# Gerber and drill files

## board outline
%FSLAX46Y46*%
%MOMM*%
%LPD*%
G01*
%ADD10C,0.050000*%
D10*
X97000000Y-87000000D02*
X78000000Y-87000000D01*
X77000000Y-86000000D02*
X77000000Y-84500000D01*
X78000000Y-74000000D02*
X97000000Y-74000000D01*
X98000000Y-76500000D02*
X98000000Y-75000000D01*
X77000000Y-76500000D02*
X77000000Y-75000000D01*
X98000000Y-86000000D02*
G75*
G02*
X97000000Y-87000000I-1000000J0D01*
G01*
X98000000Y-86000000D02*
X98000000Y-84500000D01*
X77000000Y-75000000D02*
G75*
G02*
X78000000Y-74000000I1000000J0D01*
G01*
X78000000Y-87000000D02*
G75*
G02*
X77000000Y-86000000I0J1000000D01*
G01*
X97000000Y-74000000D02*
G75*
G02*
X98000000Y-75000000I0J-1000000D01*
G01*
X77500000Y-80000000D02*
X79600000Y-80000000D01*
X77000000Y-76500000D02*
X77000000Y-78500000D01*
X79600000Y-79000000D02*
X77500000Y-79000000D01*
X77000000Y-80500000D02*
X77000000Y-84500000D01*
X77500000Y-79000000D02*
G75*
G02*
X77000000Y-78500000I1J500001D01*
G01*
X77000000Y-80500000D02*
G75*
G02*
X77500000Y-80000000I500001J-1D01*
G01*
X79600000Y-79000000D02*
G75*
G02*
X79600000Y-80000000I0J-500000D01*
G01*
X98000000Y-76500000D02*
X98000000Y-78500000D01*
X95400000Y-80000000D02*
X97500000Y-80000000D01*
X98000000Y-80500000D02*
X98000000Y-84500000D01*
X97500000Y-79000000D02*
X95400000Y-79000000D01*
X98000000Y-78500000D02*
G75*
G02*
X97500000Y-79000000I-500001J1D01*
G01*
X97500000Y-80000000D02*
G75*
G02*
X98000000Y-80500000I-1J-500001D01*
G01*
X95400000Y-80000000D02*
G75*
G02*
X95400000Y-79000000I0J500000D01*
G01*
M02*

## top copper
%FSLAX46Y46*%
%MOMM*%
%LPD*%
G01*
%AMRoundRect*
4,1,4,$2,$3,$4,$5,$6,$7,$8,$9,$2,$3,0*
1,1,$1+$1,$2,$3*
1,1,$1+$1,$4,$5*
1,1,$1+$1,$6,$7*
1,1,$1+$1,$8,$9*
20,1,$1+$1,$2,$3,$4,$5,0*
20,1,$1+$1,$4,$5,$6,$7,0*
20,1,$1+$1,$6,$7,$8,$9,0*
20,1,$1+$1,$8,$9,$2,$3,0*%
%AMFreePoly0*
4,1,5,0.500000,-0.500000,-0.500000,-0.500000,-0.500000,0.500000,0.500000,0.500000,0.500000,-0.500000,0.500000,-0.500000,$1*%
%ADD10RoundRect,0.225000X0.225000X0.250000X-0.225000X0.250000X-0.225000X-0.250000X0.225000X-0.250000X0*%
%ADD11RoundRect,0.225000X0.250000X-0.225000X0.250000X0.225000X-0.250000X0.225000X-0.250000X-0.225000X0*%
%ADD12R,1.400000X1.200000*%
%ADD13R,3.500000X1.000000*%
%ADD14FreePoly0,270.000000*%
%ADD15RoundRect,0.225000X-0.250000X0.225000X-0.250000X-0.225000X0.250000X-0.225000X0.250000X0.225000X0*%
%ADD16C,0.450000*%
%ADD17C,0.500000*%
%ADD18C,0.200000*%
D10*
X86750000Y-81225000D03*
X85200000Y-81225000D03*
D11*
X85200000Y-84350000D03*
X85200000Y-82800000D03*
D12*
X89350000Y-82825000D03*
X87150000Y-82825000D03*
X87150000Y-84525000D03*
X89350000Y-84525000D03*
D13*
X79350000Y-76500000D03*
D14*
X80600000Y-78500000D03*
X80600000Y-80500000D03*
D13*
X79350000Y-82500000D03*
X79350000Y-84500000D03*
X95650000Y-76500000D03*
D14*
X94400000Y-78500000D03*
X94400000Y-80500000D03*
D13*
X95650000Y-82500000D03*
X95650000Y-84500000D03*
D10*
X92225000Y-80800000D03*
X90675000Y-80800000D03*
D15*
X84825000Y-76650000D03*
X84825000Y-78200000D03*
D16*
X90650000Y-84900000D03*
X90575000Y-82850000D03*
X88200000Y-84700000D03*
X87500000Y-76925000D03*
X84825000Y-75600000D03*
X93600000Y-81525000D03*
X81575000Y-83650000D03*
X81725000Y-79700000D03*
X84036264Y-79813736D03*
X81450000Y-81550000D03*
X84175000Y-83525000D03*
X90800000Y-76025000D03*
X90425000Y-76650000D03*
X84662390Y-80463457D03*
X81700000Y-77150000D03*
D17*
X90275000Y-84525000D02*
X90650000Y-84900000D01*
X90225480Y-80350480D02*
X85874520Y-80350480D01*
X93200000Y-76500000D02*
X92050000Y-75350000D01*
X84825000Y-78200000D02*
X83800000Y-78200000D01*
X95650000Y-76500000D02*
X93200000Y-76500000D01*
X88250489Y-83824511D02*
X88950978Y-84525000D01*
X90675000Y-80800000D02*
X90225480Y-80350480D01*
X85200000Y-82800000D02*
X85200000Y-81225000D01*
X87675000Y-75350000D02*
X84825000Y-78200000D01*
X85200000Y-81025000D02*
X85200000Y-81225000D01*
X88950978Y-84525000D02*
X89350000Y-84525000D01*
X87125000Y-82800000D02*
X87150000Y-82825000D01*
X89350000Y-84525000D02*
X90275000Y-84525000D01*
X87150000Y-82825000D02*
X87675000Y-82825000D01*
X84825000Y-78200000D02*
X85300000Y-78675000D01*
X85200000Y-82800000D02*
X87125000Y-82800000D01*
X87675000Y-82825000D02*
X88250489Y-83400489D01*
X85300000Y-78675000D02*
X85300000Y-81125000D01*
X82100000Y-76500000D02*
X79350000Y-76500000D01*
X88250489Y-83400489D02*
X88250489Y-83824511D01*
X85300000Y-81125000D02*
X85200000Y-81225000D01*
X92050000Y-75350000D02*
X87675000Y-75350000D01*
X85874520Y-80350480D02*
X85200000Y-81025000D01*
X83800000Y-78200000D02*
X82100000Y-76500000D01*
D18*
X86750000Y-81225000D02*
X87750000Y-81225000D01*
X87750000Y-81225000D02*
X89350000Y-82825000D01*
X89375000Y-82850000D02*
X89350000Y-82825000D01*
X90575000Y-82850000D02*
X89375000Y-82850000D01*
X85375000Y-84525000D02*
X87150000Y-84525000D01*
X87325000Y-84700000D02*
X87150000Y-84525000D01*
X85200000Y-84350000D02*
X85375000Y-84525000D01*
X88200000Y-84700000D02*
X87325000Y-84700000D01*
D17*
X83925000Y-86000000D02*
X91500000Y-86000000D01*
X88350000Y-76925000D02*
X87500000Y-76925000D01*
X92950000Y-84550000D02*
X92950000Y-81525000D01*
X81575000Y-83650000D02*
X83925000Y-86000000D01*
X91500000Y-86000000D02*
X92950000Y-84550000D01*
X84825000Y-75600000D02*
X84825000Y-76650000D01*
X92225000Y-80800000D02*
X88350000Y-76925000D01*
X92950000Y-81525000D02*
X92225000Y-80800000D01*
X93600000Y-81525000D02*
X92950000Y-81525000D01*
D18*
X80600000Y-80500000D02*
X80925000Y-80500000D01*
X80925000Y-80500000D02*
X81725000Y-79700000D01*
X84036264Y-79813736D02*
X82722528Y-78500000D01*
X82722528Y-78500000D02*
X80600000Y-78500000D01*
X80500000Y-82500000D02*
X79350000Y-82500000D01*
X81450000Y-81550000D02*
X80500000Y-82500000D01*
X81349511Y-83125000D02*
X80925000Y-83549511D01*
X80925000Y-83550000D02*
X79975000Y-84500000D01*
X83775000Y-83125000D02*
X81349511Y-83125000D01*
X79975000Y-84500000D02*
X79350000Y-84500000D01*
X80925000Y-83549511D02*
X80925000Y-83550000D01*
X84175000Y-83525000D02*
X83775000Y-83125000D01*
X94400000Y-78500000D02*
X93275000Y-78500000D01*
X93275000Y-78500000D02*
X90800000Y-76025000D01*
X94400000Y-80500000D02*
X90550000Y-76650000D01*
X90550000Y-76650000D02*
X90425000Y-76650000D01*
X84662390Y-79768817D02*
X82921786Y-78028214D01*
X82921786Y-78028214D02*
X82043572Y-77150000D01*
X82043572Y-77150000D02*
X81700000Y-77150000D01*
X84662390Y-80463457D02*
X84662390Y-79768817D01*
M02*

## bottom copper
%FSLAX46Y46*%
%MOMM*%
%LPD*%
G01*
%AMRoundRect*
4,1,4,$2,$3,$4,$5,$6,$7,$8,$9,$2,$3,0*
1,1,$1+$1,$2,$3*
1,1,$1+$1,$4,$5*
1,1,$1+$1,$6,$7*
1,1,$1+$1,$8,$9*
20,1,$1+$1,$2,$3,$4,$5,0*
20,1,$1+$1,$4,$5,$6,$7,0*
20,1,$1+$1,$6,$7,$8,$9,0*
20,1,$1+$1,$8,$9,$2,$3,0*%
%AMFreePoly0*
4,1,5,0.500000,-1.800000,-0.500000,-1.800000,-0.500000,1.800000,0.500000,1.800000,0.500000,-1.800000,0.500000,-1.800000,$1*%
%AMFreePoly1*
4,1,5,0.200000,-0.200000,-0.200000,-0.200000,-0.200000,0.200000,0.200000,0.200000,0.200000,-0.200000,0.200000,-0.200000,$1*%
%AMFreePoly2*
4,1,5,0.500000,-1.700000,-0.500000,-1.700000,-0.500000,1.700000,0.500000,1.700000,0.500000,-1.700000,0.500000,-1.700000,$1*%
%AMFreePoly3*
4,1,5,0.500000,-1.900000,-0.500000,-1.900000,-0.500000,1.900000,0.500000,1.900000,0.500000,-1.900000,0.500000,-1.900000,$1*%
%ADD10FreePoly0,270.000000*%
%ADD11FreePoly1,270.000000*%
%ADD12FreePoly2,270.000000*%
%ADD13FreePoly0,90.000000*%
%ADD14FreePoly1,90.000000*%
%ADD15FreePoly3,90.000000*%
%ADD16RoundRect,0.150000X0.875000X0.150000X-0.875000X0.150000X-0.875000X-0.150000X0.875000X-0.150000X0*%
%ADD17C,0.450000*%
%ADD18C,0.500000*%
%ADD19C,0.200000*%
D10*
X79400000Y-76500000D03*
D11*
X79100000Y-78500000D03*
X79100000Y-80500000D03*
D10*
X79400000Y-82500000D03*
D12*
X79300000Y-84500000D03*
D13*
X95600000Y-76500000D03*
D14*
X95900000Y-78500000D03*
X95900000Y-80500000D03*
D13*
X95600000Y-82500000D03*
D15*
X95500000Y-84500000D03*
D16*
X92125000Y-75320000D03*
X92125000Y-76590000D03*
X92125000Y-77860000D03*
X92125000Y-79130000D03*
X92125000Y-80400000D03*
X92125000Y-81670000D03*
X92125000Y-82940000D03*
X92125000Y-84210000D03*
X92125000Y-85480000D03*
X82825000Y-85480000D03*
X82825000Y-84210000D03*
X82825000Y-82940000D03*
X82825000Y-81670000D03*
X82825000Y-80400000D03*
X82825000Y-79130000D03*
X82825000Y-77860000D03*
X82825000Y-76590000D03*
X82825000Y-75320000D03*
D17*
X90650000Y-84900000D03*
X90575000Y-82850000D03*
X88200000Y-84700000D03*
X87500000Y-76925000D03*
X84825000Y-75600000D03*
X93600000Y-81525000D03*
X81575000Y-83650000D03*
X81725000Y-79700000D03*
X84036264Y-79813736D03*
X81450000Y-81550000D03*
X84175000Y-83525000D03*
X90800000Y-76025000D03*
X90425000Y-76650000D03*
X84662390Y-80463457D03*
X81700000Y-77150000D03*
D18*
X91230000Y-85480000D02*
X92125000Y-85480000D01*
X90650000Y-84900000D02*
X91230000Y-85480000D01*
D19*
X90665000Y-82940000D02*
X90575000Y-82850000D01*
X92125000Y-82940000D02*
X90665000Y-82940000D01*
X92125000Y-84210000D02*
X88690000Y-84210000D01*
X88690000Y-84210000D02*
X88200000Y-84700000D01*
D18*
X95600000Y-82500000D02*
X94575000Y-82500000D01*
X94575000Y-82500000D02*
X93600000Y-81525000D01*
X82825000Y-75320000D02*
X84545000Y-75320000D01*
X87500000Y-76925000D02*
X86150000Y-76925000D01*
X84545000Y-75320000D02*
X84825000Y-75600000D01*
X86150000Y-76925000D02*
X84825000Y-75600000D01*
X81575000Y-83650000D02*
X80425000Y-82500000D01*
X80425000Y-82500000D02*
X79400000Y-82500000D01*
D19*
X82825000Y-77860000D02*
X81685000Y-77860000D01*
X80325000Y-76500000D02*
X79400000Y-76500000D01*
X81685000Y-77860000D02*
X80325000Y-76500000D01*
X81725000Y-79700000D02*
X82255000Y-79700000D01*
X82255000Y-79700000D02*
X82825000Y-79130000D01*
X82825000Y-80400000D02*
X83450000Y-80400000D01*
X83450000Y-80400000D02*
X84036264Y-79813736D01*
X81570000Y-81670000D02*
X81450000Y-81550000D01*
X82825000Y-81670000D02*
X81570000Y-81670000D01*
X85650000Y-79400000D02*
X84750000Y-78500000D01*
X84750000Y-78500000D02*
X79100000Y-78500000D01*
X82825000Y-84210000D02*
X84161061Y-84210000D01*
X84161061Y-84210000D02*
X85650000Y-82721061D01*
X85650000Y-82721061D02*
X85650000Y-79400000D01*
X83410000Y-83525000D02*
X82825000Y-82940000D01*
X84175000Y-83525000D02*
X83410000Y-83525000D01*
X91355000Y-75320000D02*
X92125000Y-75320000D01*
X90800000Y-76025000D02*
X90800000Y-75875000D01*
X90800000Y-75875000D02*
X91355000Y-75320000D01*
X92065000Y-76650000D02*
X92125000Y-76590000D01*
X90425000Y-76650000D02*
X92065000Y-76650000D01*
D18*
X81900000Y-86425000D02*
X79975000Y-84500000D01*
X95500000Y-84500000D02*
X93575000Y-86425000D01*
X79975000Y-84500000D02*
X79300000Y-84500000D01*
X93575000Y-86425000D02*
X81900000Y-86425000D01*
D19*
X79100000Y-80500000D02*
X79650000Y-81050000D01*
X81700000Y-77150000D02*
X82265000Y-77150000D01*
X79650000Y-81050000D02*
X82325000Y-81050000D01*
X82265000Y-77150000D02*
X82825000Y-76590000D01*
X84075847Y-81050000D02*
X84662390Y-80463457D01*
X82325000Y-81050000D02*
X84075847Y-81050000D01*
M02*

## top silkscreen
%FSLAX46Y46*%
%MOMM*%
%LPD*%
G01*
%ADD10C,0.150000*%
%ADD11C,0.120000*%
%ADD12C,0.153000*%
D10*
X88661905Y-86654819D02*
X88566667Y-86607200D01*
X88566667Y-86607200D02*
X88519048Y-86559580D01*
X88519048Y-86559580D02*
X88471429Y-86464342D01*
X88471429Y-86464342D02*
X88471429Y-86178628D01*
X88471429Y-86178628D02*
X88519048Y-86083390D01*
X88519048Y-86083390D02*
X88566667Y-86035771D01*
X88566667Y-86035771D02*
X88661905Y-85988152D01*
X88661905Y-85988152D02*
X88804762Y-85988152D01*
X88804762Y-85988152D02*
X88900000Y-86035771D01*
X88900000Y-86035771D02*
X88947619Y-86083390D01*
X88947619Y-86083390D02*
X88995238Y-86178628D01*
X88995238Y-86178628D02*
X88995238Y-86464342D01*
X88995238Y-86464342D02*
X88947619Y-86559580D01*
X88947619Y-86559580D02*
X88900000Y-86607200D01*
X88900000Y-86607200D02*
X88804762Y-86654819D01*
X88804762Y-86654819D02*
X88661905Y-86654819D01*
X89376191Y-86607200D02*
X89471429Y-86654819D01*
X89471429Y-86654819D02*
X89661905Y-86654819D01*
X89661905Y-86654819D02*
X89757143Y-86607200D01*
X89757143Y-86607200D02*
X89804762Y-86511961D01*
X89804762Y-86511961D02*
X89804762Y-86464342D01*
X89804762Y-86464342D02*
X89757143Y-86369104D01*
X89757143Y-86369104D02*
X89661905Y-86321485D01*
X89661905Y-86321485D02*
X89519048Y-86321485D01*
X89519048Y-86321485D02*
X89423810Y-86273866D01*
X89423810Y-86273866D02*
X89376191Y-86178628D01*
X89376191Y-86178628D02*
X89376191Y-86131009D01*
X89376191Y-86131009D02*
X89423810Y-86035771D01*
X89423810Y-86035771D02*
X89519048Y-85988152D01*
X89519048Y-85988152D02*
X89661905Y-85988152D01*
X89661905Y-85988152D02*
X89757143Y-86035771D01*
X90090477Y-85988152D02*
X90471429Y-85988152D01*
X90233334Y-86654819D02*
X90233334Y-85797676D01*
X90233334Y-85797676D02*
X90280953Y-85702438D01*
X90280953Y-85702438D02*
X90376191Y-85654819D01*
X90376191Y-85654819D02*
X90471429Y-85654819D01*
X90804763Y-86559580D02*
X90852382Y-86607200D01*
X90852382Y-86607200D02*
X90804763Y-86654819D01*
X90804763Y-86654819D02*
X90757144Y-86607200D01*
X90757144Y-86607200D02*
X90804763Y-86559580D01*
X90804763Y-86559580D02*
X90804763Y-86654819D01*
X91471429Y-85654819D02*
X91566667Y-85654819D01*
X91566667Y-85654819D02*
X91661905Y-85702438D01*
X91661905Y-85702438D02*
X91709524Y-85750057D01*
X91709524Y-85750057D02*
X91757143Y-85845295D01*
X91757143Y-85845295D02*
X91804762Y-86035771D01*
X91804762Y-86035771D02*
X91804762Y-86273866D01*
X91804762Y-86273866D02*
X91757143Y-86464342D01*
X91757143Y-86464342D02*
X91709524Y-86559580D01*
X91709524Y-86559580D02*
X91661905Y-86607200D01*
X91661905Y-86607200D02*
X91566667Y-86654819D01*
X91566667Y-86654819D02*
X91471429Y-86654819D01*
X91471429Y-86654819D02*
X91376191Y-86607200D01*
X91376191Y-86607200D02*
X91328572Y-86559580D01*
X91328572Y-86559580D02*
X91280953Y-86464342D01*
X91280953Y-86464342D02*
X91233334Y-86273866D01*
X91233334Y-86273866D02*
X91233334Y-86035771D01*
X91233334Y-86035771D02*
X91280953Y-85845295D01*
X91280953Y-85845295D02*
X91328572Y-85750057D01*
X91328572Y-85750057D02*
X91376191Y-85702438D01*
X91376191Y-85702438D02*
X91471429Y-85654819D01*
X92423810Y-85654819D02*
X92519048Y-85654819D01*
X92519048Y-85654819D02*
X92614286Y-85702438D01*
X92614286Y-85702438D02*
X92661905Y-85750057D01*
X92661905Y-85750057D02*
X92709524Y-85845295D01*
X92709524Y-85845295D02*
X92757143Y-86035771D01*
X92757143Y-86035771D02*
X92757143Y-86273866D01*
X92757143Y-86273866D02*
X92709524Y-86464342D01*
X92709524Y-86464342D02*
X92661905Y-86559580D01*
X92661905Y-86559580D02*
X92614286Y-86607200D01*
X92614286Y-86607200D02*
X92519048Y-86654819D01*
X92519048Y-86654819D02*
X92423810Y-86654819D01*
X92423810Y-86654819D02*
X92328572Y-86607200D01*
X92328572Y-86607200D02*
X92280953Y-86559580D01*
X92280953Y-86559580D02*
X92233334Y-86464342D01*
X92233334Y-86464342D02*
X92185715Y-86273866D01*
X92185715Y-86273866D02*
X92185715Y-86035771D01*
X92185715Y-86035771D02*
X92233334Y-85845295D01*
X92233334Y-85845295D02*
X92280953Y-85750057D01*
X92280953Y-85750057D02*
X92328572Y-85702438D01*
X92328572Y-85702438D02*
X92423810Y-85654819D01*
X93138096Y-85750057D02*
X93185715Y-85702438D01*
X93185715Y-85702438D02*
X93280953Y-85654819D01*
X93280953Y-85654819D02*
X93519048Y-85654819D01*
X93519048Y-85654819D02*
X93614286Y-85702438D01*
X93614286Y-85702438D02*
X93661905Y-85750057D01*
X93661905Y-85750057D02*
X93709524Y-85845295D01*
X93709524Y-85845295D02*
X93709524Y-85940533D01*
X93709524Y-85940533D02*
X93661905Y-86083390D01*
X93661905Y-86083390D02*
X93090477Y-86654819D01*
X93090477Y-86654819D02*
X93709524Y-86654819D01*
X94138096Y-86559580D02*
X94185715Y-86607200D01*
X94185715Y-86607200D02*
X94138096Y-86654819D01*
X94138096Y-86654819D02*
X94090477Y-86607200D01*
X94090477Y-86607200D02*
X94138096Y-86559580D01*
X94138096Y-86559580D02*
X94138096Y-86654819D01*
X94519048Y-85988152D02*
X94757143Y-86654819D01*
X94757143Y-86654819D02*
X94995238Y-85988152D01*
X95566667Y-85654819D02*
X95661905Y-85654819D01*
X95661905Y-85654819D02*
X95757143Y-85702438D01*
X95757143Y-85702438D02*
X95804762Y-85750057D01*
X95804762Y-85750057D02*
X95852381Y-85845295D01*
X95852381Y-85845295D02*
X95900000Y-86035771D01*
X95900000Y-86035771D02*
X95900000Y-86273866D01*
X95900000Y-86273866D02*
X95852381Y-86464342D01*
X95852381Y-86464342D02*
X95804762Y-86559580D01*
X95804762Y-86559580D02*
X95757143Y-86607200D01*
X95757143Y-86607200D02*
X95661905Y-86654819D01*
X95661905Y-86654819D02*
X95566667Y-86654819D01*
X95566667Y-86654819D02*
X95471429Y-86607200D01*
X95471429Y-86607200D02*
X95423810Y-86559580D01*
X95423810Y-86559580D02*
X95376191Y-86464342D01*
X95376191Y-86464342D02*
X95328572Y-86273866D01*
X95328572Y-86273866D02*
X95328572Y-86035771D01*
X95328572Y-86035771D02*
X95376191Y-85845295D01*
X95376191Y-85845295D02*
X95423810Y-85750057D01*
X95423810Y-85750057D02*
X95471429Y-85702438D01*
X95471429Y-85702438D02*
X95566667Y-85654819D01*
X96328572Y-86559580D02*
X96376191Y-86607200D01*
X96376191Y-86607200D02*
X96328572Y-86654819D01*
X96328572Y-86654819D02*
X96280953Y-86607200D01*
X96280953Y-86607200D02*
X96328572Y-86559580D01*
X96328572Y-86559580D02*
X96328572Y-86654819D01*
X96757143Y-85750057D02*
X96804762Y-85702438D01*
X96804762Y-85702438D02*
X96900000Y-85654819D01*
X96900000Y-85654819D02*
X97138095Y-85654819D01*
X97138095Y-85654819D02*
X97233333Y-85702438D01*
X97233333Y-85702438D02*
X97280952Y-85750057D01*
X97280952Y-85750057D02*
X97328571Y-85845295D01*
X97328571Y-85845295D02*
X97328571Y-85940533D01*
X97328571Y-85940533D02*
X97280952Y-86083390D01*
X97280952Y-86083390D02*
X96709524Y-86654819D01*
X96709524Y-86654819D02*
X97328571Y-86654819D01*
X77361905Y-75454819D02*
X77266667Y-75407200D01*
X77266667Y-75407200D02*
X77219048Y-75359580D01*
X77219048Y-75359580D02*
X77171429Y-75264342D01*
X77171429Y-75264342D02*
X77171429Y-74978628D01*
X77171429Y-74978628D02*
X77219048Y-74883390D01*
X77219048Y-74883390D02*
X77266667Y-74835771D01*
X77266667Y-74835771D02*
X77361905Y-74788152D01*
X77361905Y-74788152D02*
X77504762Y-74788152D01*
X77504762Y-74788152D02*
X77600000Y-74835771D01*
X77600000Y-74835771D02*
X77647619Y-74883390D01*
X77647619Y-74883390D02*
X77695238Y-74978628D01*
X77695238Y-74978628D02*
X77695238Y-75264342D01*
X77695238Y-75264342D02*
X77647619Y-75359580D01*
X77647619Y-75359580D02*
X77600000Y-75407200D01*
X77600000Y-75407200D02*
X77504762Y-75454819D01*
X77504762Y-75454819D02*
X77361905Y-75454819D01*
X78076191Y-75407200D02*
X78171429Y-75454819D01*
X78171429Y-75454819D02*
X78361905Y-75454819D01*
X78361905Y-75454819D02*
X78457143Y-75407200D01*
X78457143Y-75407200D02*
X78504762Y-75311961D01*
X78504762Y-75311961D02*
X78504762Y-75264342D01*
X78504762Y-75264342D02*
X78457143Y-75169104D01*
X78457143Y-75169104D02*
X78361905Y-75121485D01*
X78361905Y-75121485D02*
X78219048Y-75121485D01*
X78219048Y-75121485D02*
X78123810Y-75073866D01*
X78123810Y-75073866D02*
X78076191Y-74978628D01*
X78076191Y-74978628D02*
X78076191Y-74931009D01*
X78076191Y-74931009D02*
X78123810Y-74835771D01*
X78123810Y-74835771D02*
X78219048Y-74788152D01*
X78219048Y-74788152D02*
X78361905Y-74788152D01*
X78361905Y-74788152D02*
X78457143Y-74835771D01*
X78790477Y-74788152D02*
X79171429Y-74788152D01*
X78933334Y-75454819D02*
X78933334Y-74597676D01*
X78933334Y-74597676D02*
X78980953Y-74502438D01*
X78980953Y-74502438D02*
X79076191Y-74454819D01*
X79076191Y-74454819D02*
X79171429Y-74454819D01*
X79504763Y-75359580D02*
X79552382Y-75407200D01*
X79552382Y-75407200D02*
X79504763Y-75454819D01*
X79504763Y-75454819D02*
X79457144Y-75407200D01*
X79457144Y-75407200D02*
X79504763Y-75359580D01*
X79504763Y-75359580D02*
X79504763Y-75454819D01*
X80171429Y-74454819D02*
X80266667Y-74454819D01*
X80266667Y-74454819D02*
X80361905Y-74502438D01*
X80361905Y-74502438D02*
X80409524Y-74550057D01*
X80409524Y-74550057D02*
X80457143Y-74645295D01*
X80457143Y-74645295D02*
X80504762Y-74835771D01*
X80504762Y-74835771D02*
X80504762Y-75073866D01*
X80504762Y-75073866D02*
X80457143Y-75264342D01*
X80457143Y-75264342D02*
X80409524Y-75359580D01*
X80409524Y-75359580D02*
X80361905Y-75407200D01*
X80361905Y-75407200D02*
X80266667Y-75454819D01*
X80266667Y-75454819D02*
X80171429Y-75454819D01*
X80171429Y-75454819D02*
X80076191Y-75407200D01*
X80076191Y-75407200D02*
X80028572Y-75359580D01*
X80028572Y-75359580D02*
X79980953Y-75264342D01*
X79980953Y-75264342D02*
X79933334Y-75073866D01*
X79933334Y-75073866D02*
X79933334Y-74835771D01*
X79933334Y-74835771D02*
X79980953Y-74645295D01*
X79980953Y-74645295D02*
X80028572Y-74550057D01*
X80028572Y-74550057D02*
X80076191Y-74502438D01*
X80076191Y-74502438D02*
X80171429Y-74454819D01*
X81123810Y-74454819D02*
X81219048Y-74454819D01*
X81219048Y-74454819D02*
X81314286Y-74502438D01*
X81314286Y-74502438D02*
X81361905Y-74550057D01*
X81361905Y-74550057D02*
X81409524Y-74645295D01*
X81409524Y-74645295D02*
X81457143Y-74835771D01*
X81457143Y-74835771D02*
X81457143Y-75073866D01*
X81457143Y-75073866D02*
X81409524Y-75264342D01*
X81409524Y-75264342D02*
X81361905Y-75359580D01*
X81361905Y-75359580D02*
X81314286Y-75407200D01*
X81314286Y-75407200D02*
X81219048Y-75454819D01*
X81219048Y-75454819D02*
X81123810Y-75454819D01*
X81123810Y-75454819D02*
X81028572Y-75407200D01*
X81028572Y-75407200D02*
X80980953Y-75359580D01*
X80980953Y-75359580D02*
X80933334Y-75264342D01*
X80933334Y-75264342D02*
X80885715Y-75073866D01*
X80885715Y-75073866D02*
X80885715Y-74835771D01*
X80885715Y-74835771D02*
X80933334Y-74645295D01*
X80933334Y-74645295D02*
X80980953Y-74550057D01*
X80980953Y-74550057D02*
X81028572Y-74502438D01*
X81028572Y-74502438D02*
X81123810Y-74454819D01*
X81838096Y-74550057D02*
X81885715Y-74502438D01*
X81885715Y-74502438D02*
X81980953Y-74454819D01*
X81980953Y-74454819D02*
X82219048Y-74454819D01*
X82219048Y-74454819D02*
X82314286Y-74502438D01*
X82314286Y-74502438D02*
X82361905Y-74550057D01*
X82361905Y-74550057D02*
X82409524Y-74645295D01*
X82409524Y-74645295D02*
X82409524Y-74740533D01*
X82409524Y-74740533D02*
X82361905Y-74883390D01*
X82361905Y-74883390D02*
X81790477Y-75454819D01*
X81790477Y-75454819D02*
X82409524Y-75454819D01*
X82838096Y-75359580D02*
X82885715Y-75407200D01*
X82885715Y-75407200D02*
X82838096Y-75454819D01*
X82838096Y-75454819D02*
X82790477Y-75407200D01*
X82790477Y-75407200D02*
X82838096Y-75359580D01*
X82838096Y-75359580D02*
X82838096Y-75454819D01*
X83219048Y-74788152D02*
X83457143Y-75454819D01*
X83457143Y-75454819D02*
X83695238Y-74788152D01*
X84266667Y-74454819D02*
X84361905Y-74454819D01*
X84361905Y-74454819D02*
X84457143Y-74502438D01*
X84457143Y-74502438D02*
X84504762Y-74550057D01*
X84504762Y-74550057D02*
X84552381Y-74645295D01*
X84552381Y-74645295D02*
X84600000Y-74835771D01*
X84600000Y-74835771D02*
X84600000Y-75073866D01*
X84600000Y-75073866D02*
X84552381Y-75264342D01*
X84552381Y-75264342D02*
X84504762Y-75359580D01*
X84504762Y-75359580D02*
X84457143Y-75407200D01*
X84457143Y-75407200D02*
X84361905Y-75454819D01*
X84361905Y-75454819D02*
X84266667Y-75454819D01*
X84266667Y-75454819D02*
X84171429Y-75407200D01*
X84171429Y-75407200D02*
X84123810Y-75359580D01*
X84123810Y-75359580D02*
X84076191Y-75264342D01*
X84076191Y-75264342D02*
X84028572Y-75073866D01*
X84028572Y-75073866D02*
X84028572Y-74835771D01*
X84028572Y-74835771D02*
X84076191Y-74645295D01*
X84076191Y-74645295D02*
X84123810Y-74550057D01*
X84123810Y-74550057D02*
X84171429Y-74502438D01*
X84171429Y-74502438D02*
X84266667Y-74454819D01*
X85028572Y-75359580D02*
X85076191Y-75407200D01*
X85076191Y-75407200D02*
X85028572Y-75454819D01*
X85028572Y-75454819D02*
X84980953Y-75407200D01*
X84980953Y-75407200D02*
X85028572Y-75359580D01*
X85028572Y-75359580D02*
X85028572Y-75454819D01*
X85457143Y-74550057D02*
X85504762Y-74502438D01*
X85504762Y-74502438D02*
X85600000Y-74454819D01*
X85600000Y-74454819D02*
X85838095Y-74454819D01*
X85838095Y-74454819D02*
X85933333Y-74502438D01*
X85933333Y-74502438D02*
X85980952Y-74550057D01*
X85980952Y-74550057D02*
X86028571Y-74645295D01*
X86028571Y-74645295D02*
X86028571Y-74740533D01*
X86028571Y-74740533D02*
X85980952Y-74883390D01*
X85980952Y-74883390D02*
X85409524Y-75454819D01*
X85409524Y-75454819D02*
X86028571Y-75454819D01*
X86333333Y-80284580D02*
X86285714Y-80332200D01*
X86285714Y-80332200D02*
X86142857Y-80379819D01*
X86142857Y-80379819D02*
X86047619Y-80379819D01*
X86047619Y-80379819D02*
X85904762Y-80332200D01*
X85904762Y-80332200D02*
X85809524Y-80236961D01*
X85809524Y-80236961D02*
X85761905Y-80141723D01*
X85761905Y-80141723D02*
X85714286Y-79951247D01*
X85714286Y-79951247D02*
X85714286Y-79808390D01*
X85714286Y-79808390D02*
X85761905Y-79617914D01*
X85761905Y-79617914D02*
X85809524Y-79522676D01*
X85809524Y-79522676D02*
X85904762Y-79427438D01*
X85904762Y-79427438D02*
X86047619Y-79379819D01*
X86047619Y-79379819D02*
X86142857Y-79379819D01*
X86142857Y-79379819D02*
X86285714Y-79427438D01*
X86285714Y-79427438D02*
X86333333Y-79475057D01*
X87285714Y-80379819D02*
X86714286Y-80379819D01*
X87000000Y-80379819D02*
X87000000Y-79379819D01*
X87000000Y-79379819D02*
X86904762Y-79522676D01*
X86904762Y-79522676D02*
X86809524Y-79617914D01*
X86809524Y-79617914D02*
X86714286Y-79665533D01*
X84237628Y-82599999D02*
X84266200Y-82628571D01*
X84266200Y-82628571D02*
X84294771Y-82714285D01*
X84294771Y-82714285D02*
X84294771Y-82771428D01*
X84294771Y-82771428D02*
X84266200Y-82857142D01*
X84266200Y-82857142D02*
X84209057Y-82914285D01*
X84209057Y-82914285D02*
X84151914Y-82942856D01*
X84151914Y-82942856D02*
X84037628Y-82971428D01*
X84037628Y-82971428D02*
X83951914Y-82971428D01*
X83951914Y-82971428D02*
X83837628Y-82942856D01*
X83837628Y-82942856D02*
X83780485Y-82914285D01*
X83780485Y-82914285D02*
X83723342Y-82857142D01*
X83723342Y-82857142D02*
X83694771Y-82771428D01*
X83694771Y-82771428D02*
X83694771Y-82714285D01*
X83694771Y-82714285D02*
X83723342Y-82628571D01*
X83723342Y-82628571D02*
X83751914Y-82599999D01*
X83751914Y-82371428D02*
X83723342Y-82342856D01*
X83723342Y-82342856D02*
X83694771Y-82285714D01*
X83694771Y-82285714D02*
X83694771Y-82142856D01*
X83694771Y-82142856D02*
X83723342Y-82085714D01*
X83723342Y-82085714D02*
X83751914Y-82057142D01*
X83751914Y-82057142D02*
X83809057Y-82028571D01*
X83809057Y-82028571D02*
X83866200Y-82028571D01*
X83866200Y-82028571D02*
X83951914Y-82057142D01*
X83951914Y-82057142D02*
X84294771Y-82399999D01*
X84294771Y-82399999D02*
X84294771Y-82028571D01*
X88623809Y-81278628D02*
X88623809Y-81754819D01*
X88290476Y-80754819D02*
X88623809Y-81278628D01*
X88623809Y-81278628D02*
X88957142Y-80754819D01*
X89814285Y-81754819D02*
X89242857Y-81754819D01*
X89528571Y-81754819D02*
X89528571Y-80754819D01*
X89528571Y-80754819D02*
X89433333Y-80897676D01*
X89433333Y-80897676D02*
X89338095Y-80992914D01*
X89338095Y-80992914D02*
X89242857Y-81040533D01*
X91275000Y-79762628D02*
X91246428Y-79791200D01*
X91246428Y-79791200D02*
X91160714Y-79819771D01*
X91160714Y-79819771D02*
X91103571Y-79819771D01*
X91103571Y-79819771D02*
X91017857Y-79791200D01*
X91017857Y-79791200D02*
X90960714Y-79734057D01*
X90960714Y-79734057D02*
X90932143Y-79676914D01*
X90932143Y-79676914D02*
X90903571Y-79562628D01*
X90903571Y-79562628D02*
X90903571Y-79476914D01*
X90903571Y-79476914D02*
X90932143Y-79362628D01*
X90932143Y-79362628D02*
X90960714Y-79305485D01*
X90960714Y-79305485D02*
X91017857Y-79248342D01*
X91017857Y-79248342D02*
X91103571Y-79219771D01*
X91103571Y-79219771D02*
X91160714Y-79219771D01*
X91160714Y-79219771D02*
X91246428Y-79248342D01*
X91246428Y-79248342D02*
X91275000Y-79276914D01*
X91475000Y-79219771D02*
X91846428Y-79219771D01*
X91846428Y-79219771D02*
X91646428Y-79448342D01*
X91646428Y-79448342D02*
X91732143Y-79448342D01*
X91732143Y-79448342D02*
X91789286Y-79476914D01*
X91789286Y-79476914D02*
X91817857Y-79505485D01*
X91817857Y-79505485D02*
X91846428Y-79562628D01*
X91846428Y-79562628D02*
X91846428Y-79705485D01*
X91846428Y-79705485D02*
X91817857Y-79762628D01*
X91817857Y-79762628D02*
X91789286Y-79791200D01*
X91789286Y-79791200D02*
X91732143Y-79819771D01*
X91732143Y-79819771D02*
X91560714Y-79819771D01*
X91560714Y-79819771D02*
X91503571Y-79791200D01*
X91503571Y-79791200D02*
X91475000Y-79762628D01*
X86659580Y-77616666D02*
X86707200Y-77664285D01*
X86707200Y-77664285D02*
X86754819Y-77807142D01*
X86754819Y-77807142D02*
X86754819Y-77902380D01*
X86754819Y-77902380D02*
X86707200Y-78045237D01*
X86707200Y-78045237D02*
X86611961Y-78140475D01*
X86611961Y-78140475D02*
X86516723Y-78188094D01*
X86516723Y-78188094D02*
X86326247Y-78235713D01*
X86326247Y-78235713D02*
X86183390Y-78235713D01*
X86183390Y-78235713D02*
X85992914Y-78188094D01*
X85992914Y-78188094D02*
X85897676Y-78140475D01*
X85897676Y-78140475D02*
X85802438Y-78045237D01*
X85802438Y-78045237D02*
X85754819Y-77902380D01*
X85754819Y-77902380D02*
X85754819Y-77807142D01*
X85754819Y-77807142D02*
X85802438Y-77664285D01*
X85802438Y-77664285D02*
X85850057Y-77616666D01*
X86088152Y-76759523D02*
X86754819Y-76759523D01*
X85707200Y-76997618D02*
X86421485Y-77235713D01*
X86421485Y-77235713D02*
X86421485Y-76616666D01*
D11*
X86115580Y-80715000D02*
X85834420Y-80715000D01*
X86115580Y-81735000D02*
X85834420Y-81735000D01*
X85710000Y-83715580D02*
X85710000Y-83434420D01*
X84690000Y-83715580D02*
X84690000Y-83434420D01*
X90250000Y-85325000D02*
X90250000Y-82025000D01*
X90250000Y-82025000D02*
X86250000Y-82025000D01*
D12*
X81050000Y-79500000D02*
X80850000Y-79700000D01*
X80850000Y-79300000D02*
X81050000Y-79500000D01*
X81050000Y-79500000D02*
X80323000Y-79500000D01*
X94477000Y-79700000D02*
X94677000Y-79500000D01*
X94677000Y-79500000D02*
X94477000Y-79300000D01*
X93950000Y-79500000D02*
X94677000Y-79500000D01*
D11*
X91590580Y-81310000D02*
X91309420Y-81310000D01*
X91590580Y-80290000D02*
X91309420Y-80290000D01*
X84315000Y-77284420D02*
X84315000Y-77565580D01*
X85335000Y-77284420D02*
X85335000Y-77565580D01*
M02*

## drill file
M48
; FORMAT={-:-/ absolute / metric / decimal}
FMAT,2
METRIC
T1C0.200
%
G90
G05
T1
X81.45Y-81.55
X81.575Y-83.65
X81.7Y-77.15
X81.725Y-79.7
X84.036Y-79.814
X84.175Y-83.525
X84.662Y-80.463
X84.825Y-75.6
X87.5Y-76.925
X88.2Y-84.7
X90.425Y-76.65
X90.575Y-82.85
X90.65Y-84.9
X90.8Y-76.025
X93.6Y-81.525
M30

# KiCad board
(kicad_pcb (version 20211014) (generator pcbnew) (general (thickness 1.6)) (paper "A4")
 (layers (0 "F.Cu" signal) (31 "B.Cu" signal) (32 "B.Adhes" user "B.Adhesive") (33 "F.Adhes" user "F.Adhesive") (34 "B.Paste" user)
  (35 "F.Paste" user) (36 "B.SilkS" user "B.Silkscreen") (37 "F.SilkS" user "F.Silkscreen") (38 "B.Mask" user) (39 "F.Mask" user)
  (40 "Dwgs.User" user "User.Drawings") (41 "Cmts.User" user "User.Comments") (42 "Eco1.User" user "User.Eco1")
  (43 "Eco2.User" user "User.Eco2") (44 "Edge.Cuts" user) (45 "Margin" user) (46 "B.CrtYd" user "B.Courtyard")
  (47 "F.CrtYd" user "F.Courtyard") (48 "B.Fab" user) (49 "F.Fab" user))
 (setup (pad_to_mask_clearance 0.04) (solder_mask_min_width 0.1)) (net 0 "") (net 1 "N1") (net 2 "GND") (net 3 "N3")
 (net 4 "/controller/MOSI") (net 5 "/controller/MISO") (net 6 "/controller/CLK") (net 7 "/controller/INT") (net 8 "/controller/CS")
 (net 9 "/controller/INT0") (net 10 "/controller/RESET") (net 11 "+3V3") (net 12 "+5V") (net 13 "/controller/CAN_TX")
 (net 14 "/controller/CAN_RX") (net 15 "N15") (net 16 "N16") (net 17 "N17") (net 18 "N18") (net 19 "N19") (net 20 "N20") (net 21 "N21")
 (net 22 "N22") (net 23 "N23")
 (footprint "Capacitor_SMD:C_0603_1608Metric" (layer "F.Cu") (at 85.975 81.225 180)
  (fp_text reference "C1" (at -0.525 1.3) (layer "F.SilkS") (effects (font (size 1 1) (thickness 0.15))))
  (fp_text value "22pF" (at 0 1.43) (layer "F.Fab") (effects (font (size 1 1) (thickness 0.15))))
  (fp_line (start -0.14058 0.51) (end 0.14058 0.51) (layer "F.SilkS") (width 0.12))
  (fp_line (start -0.14058 -0.51) (end 0.14058 -0.51) (layer "F.SilkS") (width 0.12))
  (pad "1" smd roundrect locked (at -0.775 0 180) (size 0.9 0.95) (layers "F.Cu" "F.Paste" "F.Mask") (roundrect_rratio 0.25) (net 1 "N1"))
  (pad "2" smd roundrect locked (at 0.775 0 180) (size 0.9 0.95) (layers "F.Cu" "F.Paste" "F.Mask") (roundrect_rratio 0.25) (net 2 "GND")))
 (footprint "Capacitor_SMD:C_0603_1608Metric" (layer "F.Cu") (at 85.2 83.575 90)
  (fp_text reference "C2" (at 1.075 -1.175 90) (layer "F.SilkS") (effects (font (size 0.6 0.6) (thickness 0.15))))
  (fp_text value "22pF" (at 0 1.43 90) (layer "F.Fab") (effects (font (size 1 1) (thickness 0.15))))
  (fp_line (start -0.14058 0.51) (end 0.14058 0.51) (layer "F.SilkS") (width 0.12))
  (fp_line (start -0.14058 -0.51) (end 0.14058 -0.51) (layer "F.SilkS") (width 0.12))
  (pad "1" smd roundrect locked (at -0.775 0 90) (size 0.9 0.95) (layers "F.Cu" "F.Paste" "F.Mask") (roundrect_rratio 0.25) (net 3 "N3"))
  (pad "2" smd roundrect locked (at 0.775 0 90) (size 0.9 0.95) (layers "F.Cu" "F.Paste" "F.Mask") (roundrect_rratio 0.25) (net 2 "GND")))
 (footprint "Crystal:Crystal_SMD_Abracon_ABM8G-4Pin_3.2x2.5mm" (layer "F.Cu") (at 88.25 83.675 180)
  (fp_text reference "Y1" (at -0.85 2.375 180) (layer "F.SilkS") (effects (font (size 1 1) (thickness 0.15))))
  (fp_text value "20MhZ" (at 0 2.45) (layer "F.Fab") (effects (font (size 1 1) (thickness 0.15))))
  (fp_line (start -2 -1.65) (end -2 1.65) (layer "F.SilkS") (width 0.12))
  (fp_line (start -2 1.65) (end 2 1.65) (layer "F.SilkS") (width 0.12))
  (pad "1" smd rect locked (at -1.1 0.85 180) (size 1.4 1.2) (layers "F.Cu" "F.Paste" "F.Mask") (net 1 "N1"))
  (pad "2" smd rect locked (at 1.1 0.85 180) (size 1.4 1.2) (layers "F.Cu" "F.Paste" "F.Mask") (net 2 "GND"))
  (pad "3" smd rect locked (at 1.1 -0.85 180) (size 1.4 1.2) (layers "F.Cu" "F.Paste" "F.Mask") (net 3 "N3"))
  (pad "4" smd rect locked (at -1.1 -0.85 180) (size 1.4 1.2) (layers "F.Cu" "F.Paste" "F.Mask") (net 2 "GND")))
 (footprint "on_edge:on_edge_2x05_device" (layer "F.Cu") (at 77 80.5 -90)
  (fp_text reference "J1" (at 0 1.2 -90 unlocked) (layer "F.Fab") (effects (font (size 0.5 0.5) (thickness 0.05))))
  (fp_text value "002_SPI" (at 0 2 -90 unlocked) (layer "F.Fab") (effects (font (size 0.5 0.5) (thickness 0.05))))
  (fp_line (start -1 -4.05) (end -0.8 -3.85) (layer "F.SilkS") (width 0.153))
  (fp_line (start -1.2 -3.85) (end -1 -4.05) (layer "F.SilkS") (width 0.153))
  (fp_line (start -1 -4.05) (end -1 -3.323) (layer "F.SilkS") (width 0.153))
  (fp_line (start -0.5 -0.5) (end -0.5 -2.6) (layer "Edge.Cuts") (width 0.05))
  (fp_line (start -4 0) (end -2 0) (layer "Edge.Cuts") (width 0.05))
  (fp_line (start -1.5 -2.6) (end -1.5 -0.5) (layer "Edge.Cuts") (width 0.05))
  (fp_line (start 0 0) (end 4 0) (layer "Edge.Cuts") (width 0.05))
  (fp_arc (start -1.5 -0.5) (mid -1.646447 -0.146447) (end -2 0) (layer "Edge.Cuts") (width 0.05))
  (fp_arc (start 0 0) (mid -0.353553 -0.146447) (end -0.5 -0.5) (layer "Edge.Cuts") (width 0.05))
  (fp_arc (start -1.5 -2.6) (mid -1 -3.1) (end -0.5 -2.6) (layer "Edge.Cuts") (width 0.05))
  (pad "1" smd rect locked (at -4 -2.35 90) (size 1 3.5) (layers "F.Cu" "F.Mask") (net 2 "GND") (zone_connect 0))
  (pad "2" smd custom locked (at -2 -3.6 270) (size 1 1) (layers "F.Cu" "F.Mask") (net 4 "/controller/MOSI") (zone_connect 0)
   (options (clearance outline) (anchor rect)) (primitives))
  (pad "3" smd custom locked (at 0 -3.6 270) (size 1 1) (layers "F.Cu" "F.Mask") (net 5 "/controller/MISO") (zone_connect 0)
   (options (clearance outline) (anchor rect)) (primitives))
  (pad "4" smd rect locked (at 2 -2.35 90) (size 1 3.5) (layers "F.Cu" "F.Mask") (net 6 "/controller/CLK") (zone_connect 0))
  (pad "5" smd rect locked (at 4 -2.35 90) (size 1 3.5) (layers "F.Cu" "F.Mask") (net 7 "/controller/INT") (zone_connect 0))
  (pad "6" smd custom locked (at -4 -2.4 270) (size 1 3.6) (layers "B.Cu" "B.Mask") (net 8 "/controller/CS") (zone_connect 0)
   (options (clearance outline) (anchor rect)) (primitives))
  (pad "7" smd custom locked (at -2 -2.1 270) (size 0.4 0.4) (layers "B.Cu" "B.Mask") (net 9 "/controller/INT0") (zone_connect 0)
   (options (clearance outline) (anchor rect)) (primitives))
  (pad "8" smd custom locked (at 0 -2.1 270) (size 0.4 0.4) (layers "B.Cu" "B.Mask") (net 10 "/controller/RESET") (zone_connect 0)
   (options (clearance outline) (anchor rect)) (primitives))
  (pad "9" smd custom locked (at 2 -2.4 270) (size 1 3.6) (layers "B.Cu" "B.Mask") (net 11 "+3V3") (zone_connect 0)
   (options (clearance outline) (anchor rect)) (primitives))
  (pad "10" smd custom locked (at 4 -2.3 270) (size 1 3.4) (layers "B.Cu" "B.Mask") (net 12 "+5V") (zone_connect 0)
   (options (clearance outline) (anchor rect)) (primitives)))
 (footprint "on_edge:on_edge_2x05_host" (layer "F.Cu") (at 98 80.5 -90)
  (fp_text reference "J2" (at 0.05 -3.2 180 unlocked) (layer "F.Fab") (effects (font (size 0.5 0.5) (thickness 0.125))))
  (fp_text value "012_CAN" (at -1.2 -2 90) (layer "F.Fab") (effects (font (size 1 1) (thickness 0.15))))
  (fp_line (start -0.8 3.523) (end -1 3.323) (layer "F.SilkS") (width 0.153))
  (fp_line (start -1 3.323) (end -1.2 3.523) (layer "F.SilkS") (width 0.153))
  (fp_line (start -1 4.05) (end -1 3.323) (layer "F.SilkS") (width 0.153))
  (fp_line (start -4 0) (end -2 0) (layer "Edge.Cuts") (width 0.05))
  (fp_line (start -0.5 2.6) (end -0.5 0.5) (layer "Edge.Cuts") (width 0.05))
  (fp_line (start 0 0) (end 4 0) (layer "Edge.Cuts") (width 0.05))
  (fp_line (start -1.5 0.5) (end -1.5 2.6) (layer "Edge.Cuts") (width 0.05))
  (fp_arc (start -2 0) (mid -1.646447 0.146447) (end -1.5 0.5) (layer "Edge.Cuts") (width 0.05))
  (fp_arc (start -0.5 0.5) (mid -0.353553 0.146447) (end 0 0) (layer "Edge.Cuts") (width 0.05))
  (fp_arc (start -0.5 2.6) (mid -1 3.1) (end -1.5 2.6) (layer "Edge.Cuts") (width 0.05))
  (pad "1" smd rect locked (at -4 2.35 270) (size 1 3.5) (layers "F.Cu" "F.Mask") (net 2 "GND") (zone_connect 0))
  (pad "2" smd custom locked (at -2 3.6 270) (size 1 1) (layers "F.Cu" "F.Mask") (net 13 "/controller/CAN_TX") (zone_connect 0)
   (options (clearance outline) (anchor rect)) (primitives))
  (pad "3" smd custom locked (at 0 3.6 270) (size 1 1) (layers "F.Cu" "F.Mask") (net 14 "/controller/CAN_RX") (zone_connect 0)
   (options (clearance outline) (anchor rect)) (primitives))
  (pad "4" smd rect locked (at 2 2.35 270) (size 1 3.5) (layers "F.Cu" "F.Mask") (zone_connect 0))
  (pad "5" smd rect locked (at 4 2.35 270) (size 1 3.5) (layers "F.Cu" "F.Mask") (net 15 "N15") (zone_connect 0))
  (pad "6" smd custom locked (at -4 2.4 90) (size 1 3.6) (layers "B.Cu" "B.Mask") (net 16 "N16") (zone_connect 0)
   (options (clearance outline) (anchor rect)) (primitives))
  (pad "7" smd custom locked (at -2 2.1 90) (size 0.4 0.4) (layers "B.Cu" "B.Mask") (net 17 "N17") (zone_connect 0)
   (options (clearance outline) (anchor rect)) (primitives))
  (pad "8" smd custom locked (at 0 2.1 90) (size 0.4 0.4) (layers "B.Cu" "B.Mask") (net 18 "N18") (zone_connect 0)
   (options (clearance outline) (anchor rect)) (primitives))
  (pad "9" smd custom locked (at 2 2.4 90) (size 1 3.6) (layers "B.Cu" "B.Mask") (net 11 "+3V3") (zone_connect 0)
   (options (clearance outline) (anchor rect)) (primitives))
  (pad "10" smd custom locked (at 4 2.5 90) (size 1 3.8) (layers "B.Cu" "B.Mask") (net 12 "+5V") (zone_connect 0)
   (options (clearance outline) (anchor rect)) (primitives)))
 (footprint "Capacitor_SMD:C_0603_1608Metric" (layer "F.Cu") (at 91.45 80.8 180)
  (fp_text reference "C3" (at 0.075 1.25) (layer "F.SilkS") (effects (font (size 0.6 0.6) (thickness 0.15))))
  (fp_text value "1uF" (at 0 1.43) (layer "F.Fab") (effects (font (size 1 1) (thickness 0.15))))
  (fp_line (start -0.14058 -0.51) (end 0.14058 -0.51) (layer "F.SilkS") (width 0.12))
  (fp_line (start -0.14058 0.51) (end 0.14058 0.51) (layer "F.SilkS") (width 0.12))
  (pad "1" smd roundrect locked (at -0.775 0 180) (size 0.9 0.95) (layers "F.Cu" "F.Paste" "F.Mask") (roundrect_rratio 0.25) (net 11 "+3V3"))
  (pad "2" smd roundrect locked (at 0.775 0 180) (size 0.9 0.95) (layers "F.Cu" "F.Paste" "F.Mask") (roundrect_rratio 0.25) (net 2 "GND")))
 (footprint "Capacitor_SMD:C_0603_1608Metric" (layer "F.Cu") (at 84.825 77.425 -90)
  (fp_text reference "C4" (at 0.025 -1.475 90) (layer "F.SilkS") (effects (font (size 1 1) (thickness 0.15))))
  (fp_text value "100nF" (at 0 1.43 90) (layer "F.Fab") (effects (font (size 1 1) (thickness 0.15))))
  (fp_line (start -0.14058 0.51) (end 0.14058 0.51) (layer "F.SilkS") (width 0.12))
  (fp_line (start -0.14058 -0.51) (end 0.14058 -0.51) (layer "F.SilkS") (width 0.12))
  (pad "1" smd roundrect locked (at -0.775 0 270) (size 0.9 0.95) (layers "F.Cu" "F.Paste" "F.Mask") (roundrect_rratio 0.25) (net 11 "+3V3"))
  (pad "2" smd roundrect locked (at 0.775 0 270) (size 0.9 0.95) (layers "F.Cu" "F.Paste" "F.Mask") (roundrect_rratio 0.25) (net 2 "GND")))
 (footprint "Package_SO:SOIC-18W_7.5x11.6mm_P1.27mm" (layer "B.Cu") (at 87.475 80.4 180)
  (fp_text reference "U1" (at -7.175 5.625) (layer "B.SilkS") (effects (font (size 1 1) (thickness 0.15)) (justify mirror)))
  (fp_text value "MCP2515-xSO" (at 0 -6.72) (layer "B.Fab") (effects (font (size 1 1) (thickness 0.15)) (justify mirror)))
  (pad "1" smd roundrect (at -4.65 5.08 180) (size 2.05 0.6) (layers "B.Cu" "B.Paste" "B.Mask") (roundrect_rratio 0.25)
   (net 13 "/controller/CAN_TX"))
  (pad "2" smd roundrect (at -4.65 3.81 180) (size 2.05 0.6) (layers "B.Cu" "B.Paste" "B.Mask") (roundrect_rratio 0.25)
   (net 14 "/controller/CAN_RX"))
  (pad "3" smd roundrect (at -4.65 2.54 180) (size 2.05 0.6) (layers "B.Cu" "B.Paste" "B.Mask") (roundrect_rratio 0.25) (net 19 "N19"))
  (pad "4" smd roundrect (at -4.65 1.27 180) (size 2.05 0.6) (layers "B.Cu" "B.Paste" "B.Mask") (roundrect_rratio 0.25) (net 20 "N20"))
  (pad "5" smd roundrect (at -4.65 0 180) (size 2.05 0.6) (layers "B.Cu" "B.Paste" "B.Mask") (roundrect_rratio 0.25) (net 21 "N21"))
  (pad "6" smd roundrect (at -4.65 -1.27 180) (size 2.05 0.6) (layers "B.Cu" "B.Paste" "B.Mask") (roundrect_rratio 0.25) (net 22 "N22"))
  (pad "7" smd roundrect (at -4.65 -2.54 180) (size 2.05 0.6) (layers "B.Cu" "B.Paste" "B.Mask") (roundrect_rratio 0.25) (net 1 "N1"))
  (pad "8" smd roundrect (at -4.65 -3.81 180) (size 2.05 0.6) (layers "B.Cu" "B.Paste" "B.Mask") (roundrect_rratio 0.25) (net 3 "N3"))
  (pad "9" smd roundrect (at -4.65 -5.08 180) (size 2.05 0.6) (layers "B.Cu" "B.Paste" "B.Mask") (roundrect_rratio 0.25) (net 2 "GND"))
  (pad "10" smd roundrect (at 4.65 -5.08 180) (size 2.05 0.6) (layers "B.Cu" "B.Paste" "B.Mask") (roundrect_rratio 0.25) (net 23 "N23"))
  (pad "11" smd roundrect (at 4.65 -3.81 180) (size 2.05 0.6) (layers "B.Cu" "B.Paste" "B.Mask") (roundrect_rratio 0.25)
   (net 9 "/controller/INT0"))
  (pad "12" smd roundrect (at 4.65 -2.54 180) (size 2.05 0.6) (layers "B.Cu" "B.Paste" "B.Mask") (roundrect_rratio 0.25)
   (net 7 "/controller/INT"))
  (pad "13" smd roundrect (at 4.65 -1.27 180) (size 2.05 0.6) (layers "B.Cu" "B.Paste" "B.Mask") (roundrect_rratio 0.25)
   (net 6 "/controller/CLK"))
  (pad "14" smd roundrect (at 4.65 0 180) (size 2.05 0.6) (layers "B.Cu" "B.Paste" "B.Mask") (roundrect_rratio 0.25)
   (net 4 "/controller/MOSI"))
  (pad "15" smd roundrect (at 4.65 1.27 180) (size 2.05 0.6) (layers "B.Cu" "B.Paste" "B.Mask") (roundrect_rratio 0.25)
   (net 5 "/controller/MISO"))
  (pad "16" smd roundrect (at 4.65 2.54 180) (size 2.05 0.6) (layers "B.Cu" "B.Paste" "B.Mask") (roundrect_rratio 0.25)
   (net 8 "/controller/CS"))
  (pad "17" smd roundrect (at 4.65 3.81 180) (size 2.05 0.6) (layers "B.Cu" "B.Paste" "B.Mask") (roundrect_rratio 0.25)
   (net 10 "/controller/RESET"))
  (pad "18" smd roundrect (at 4.65 5.08 180) (size 2.05 0.6) (layers "B.Cu" "B.Paste" "B.Mask") (roundrect_rratio 0.25) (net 11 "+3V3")))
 (gr_line (start 97 87) (end 78 87) (layer "Edge.Cuts") (width 0.05))
 (gr_line (start 77 86) (end 77 84.5) (layer "Edge.Cuts") (width 0.05))
 (gr_line (start 78 74) (end 97 74) (layer "Edge.Cuts") (width 0.05))
 (gr_line (start 98 76.5) (end 98 75) (layer "Edge.Cuts") (width 0.05))
 (gr_line (start 77 76.5) (end 77 75) (layer "Edge.Cuts") (width 0.05))
 (gr_arc (start 98 86) (mid 97.707107 86.707107) (end 97 87) (layer "Edge.Cuts") (width 0.05))
 (gr_line (start 98 86) (end 98 84.5) (layer "Edge.Cuts") (width 0.05))
 (gr_arc (start 77 75) (mid 77.292893 74.292893) (end 78 74) (layer "Edge.Cuts") (width 0.05))
 (gr_arc (start 78 87) (mid 77.292893 86.707107) (end 77 86) (layer "Edge.Cuts") (width 0.05))
 (gr_arc (start 97 74) (mid 97.707107 74.292893) (end 98 75) (layer "Edge.Cuts") (width 0.05))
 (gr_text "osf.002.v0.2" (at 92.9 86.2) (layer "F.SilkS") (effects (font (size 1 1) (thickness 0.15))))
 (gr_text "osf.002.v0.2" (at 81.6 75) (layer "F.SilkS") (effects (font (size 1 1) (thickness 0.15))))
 (segment (start 90.275 84.525) (end 90.65 84.9) (width 0.5) (layer "F.Cu") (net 2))
 (segment (start 90.22548 80.35048) (end 85.87452 80.35048) (width 0.5) (layer "F.Cu") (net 2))
 (segment (start 93.2 76.5) (end 92.05 75.35) (width 0.5) (layer "F.Cu") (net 2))
 (segment (start 84.825 78.2) (end 83.8 78.2) (width 0.5) (layer "F.Cu") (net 2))
 (segment (start 95.65 76.5) (end 93.2 76.5) (width 0.5) (layer "F.Cu") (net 2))
 (segment (start 88.250489 83.824511) (end 88.950978 84.525) (width 0.5) (layer "F.Cu") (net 2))
 (segment (start 90.675 80.8) (end 90.22548 80.35048) (width 0.5) (layer "F.Cu") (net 2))
 (segment (start 85.2 82.8) (end 85.2 81.225) (width 0.5) (layer "F.Cu") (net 2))
 (segment (start 87.675 75.35) (end 84.825 78.2) (width 0.5) (layer "F.Cu") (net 2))
 (segment (start 85.2 81.025) (end 85.2 81.225) (width 0.5) (layer "F.Cu") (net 2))
 (segment (start 88.950978 84.525) (end 89.35 84.525) (width 0.5) (layer "F.Cu") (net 2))
 (segment (start 87.125 82.8) (end 87.15 82.825) (width 0.5) (layer "F.Cu") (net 2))
 (segment (start 89.35 84.525) (end 90.275 84.525) (width 0.5) (layer "F.Cu") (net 2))
 (segment (start 87.15 82.825) (end 87.675 82.825) (width 0.5) (layer "F.Cu") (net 2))
 (segment (start 84.825 78.2) (end 85.3 78.675) (width 0.5) (layer "F.Cu") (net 2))
 (segment (start 85.2 82.8) (end 87.125 82.8) (width 0.5) (layer "F.Cu") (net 2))
 (segment (start 87.675 82.825) (end 88.250489 83.400489) (width 0.5) (layer "F.Cu") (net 2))
 (segment (start 85.3 78.675) (end 85.3 81.125) (width 0.5) (layer "F.Cu") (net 2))
 (segment (start 82.1 76.5) (end 79.35 76.5) (width 0.5) (layer "F.Cu") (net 2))
 (segment (start 88.250489 83.400489) (end 88.250489 83.824511) (width 0.5) (layer "F.Cu") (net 2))
 (segment (start 85.3 81.125) (end 85.2 81.225) (width 0.5) (layer "F.Cu") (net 2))
 (segment (start 92.05 75.35) (end 87.675 75.35) (width 0.5) (layer "F.Cu") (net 2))
 (segment (start 85.87452 80.35048) (end 85.2 81.025) (width 0.5) (layer "F.Cu") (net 2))
 (segment (start 83.8 78.2) (end 82.1 76.5) (width 0.5) (layer "F.Cu") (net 2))
 (via (at 90.65 84.9) (size 0.45) (drill 0.2) (layers "F.Cu" "B.Cu") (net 2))
 (segment (start 91.23 85.48) (end 92.125 85.48) (width 0.5) (layer "B.Cu") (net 2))
 (segment (start 90.65 84.9) (end 91.23 85.48) (width 0.5) (layer "B.Cu") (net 2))
 (segment (start 86.75 81.225) (end 87.75 81.225) (width 0.2) (layer "F.Cu") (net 1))
 (segment (start 87.75 81.225) (end 89.35 82.825) (width 0.2) (layer "F.Cu") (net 1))
 (segment (start 89.375 82.85) (end 89.35 82.825) (width 0.2) (layer "F.Cu") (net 1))
 (segment (start 90.575 82.85) (end 89.375 82.85) (width 0.2) (layer "F.Cu") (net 1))
 (via (at 90.575 82.85) (size 0.45) (drill 0.2) (layers "F.Cu" "B.Cu") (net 1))
 (segment (start 90.665 82.94) (end 90.575 82.85) (width 0.2) (layer "B.Cu") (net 1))
 (segment (start 92.125 82.94) (end 90.665 82.94) (width 0.2) (layer "B.Cu") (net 1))
 (segment (start 85.375 84.525) (end 87.15 84.525) (width 0.2) (layer "F.Cu") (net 3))
 (segment (start 87.325 84.7) (end 87.15 84.525) (width 0.2) (layer "F.Cu") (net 3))
 (segment (start 85.2 84.35) (end 85.375 84.525) (width 0.2) (layer "F.Cu") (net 3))
 (segment (start 88.2 84.7) (end 87.325 84.7) (width 0.2) (layer "F.Cu") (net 3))
 (via (at 88.2 84.7) (size 0.45) (drill 0.2) (layers "F.Cu" "B.Cu") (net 3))
 (segment (start 92.125 84.21) (end 88.69 84.21) (width 0.2) (layer "B.Cu") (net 3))
 (segment (start 88.69 84.21) (end 88.2 84.7) (width 0.2) (layer "B.Cu") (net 3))
 (segment (start 83.925 86) (end 91.5 86) (width 0.5) (layer "F.Cu") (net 11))
 (segment (start 88.35 76.925) (end 87.5 76.925) (width 0.5) (layer "F.Cu") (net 11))
 (segment (start 92.95 84.55) (end 92.95 81.525) (width 0.5) (layer "F.Cu") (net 11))
 (segment (start 81.575 83.65) (end 83.925 86) (width 0.5) (layer "F.Cu") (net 11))
 (segment (start 91.5 86) (end 92.95 84.55) (width 0.5) (layer "F.Cu") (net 11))
 (segment (start 84.825 75.6) (end 84.825 76.65) (width 0.5) (layer "F.Cu") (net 11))
 (segment (start 92.225 80.8) (end 88.35 76.925) (width 0.5) (layer "F.Cu") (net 11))
 (segment (start 92.95 81.525) (end 92.225 80.8) (width 0.5) (layer "F.Cu") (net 11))
 (segment (start 93.6 81.525) (end 92.95 81.525) (width 0.5) (layer "F.Cu") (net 11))
 (via (at 87.5 76.925) (size 0.45) (drill 0.2) (layers "F.Cu" "B.Cu") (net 11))
 (via (at 84.825 75.6) (size 0.45) (drill 0.2) (layers "F.Cu" "B.Cu") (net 11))
 (via (at 93.6 81.525) (size 0.45) (drill 0.2) (layers "F.Cu" "B.Cu") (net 11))
 (via (at 81.575 83.65) (size 0.45) (drill 0.2) (layers "F.Cu" "B.Cu") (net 11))
 (segment (start 95.6 82.5) (end 94.575 82.5) (width 0.5) (layer "B.Cu") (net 11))
 (segment (start 94.575 82.5) (end 93.6 81.525) (width 0.5) (layer "B.Cu") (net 11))
 (segment (start 82.825 75.32) (end 84.545 75.32) (width 0.5) (layer "B.Cu") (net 11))
 (segment (start 87.5 76.925) (end 86.15 76.925) (width 0.5) (layer "B.Cu") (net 11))
 (segment (start 84.545 75.32) (end 84.825 75.6) (width 0.5) (layer "B.Cu") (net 11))
 (segment (start 86.15 76.925) (end 84.825 75.6) (width 0.5) (layer "B.Cu") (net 11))
 (segment (start 81.575 83.65) (end 80.425 82.5) (width 0.5) (layer "B.Cu") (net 11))
 (segment (start 80.425 82.5) (end 79.4 82.5) (width 0.5) (layer "B.Cu") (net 11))
 (segment (start 82.825 77.86) (end 81.685 77.86) (width 0.2) (layer "B.Cu") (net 8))
 (segment (start 80.325 76.5) (end 79.4 76.5) (width 0.2) (layer "B.Cu") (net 8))
 (segment (start 81.685 77.86) (end 80.325 76.5) (width 0.2) (layer "B.Cu") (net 8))
 (segment (start 80.6 80.5) (end 80.925 80.5) (width 0.2) (layer "F.Cu") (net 5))
 (segment (start 80.925 80.5) (end 81.725 79.7) (width 0.2) (layer "F.Cu") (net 5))
 (via (at 81.725 79.7) (size 0.45) (drill 0.2) (layers "F.Cu" "B.Cu") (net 5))
 (segment (start 81.725 79.7) (end 82.255 79.7) (width 0.2) (layer "B.Cu") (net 5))
 (segment (start 82.255 79.7) (end 82.825 79.13) (width 0.2) (layer "B.Cu") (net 5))
 (segment (start 84.036264 79.813736) (end 82.722528 78.5) (width 0.2) (layer "F.Cu") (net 4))
 (segment (start 82.722528 78.5) (end 80.6 78.5) (width 0.2) (layer "F.Cu") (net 4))
 (via (at 84.036264 79.813736) (size 0.45) (drill 0.2) (layers "F.Cu" "B.Cu") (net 4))
 (segment (start 82.825 80.4) (end 83.45 80.4) (width 0.2) (layer "B.Cu") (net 4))
 (segment (start 83.45 80.4) (end 84.036264 79.813736) (width 0.2) (layer "B.Cu") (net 4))
 (segment (start 80.5 82.5) (end 79.35 82.5) (width 0.2) (layer "F.Cu") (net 6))
 (segment (start 81.45 81.55) (end 80.5 82.5) (width 0.2) (layer "F.Cu") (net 6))
 (via (at 81.45 81.55) (size 0.45) (drill 0.2) (layers "F.Cu" "B.Cu") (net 6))
 (segment (start 81.57 81.67) (end 81.45 81.55) (width 0.2) (layer "B.Cu") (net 6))
 (segment (start 82.825 81.67) (end 81.57 81.67) (width 0.2) (layer "B.Cu") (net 6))
 (segment (start 85.65 79.4) (end 84.75 78.5) (width 0.2) (layer "B.Cu") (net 9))
 (segment (start 84.75 78.5) (end 79.1 78.5) (width 0.2) (layer "B.Cu") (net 9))
 (segment (start 82.825 84.21) (end 84.161061 84.21) (width 0.2) (layer "B.Cu") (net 9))
 (segment (start 84.161061 84.21) (end 85.65 82.721061) (width 0.2) (layer "B.Cu") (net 9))
 (segment (start 85.65 82.721061) (end 85.65 79.4) (width 0.2) (layer "B.Cu") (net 9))
 (segment (start 81.349511 83.125) (end 80.925 83.549511) (width 0.2) (layer "F.Cu") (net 7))
 (segment (start 80.925 83.55) (end 79.975 84.5) (width 0.2) (layer "F.Cu") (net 7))
 (segment (start 83.775 83.125) (end 81.349511 83.125) (width 0.2) (layer "F.Cu") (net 7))
 (segment (start 79.975 84.5) (end 79.35 84.5) (width 0.2) (layer "F.Cu") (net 7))
 (segment (start 80.925 83.549511) (end 80.925 83.55) (width 0.2) (layer "F.Cu") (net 7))
 (segment (start 84.175 83.525) (end 83.775 83.125) (width 0.2) (layer "F.Cu") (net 7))
 (via (at 84.175 83.525) (size 0.45) (drill 0.2) (layers "F.Cu" "B.Cu") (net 7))
 (segment (start 83.41 83.525) (end 82.825 82.94) (width 0.2) (layer "B.Cu") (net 7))
 (segment (start 84.175 83.525) (end 83.41 83.525) (width 0.2) (layer "B.Cu") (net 7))
 (segment (start 94.4 78.5) (end 93.275 78.5) (width 0.2) (layer "F.Cu") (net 13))
 (segment (start 93.275 78.5) (end 90.8 76.025) (width 0.2) (layer "F.Cu") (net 13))
 (via (at 90.8 76.025) (size 0.45) (drill 0.2) (layers "F.Cu" "B.Cu") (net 13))
 (segment (start 91.355 75.32) (end 92.125 75.32) (width 0.2) (layer "B.Cu") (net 13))
 (segment (start 90.8 76.025) (end 90.8 75.875) (width 0.2) (layer "B.Cu") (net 13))
 (segment (start 90.8 75.875) (end 91.355 75.32) (width 0.2) (layer "B.Cu") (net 13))
 (segment (start 94.4 80.5) (end 90.55 76.65) (width 0.2) (layer "F.Cu") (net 14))
 (segment (start 90.55 76.65) (end 90.425 76.65) (width 0.2) (layer "F.Cu") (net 14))
 (via (at 90.425 76.65) (size 0.45) (drill 0.2) (layers "F.Cu" "B.Cu") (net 14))
 (segment (start 92.065 76.65) (end 92.125 76.59) (width 0.2) (layer "B.Cu") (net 14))
 (segment (start 90.425 76.65) (end 92.065 76.65) (width 0.2) (layer "B.Cu") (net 14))
 (segment (start 81.9 86.425) (end 79.975 84.5) (width 0.5) (layer "B.Cu") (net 12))
 (segment (start 95.5 84.5) (end 93.575 86.425) (width 0.5) (layer "B.Cu") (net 12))
 (segment (start 79.975 84.5) (end 79.3 84.5) (width 0.5) (layer "B.Cu") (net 12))
 (segment (start 93.575 86.425) (end 81.9 86.425) (width 0.5) (layer "B.Cu") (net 12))
 (segment (start 84.66239 79.768817) (end 82.921786 78.028214) (width 0.2) (layer "F.Cu") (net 10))
 (segment (start 82.921786 78.028214) (end 82.043572 77.15) (width 0.2) (layer "F.Cu") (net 10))
 (segment (start 82.043572 77.15) (end 81.7 77.15) (width 0.2) (layer "F.Cu") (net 10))
 (segment (start 84.66239 80.463457) (end 84.66239 79.768817) (width 0.2) (layer "F.Cu") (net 10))
 (via (at 84.66239 80.463457) (size 0.45) (drill 0.2) (layers "F.Cu" "B.Cu") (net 10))
 (via (at 81.7 77.15) (size 0.45) (drill 0.2) (layers "F.Cu" "B.Cu") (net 10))
 (segment (start 79.1 80.5) (end 79.65 81.05) (width 0.2) (layer "B.Cu") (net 10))
 (segment (start 81.7 77.15) (end 82.265 77.15) (width 0.2) (layer "B.Cu") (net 10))
 (segment (start 79.65 81.05) (end 82.325 81.05) (width 0.2) (layer "B.Cu") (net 10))
 (segment (start 82.265 77.15) (end 82.825 76.59) (width 0.2) (layer "B.Cu") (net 10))
 (segment (start 84.075847 81.05) (end 84.66239 80.463457) (width 0.2) (layer "B.Cu") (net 10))
 (segment (start 82.325 81.05) (end 84.075847 81.05) (width 0.2) (layer "B.Cu") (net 10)))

